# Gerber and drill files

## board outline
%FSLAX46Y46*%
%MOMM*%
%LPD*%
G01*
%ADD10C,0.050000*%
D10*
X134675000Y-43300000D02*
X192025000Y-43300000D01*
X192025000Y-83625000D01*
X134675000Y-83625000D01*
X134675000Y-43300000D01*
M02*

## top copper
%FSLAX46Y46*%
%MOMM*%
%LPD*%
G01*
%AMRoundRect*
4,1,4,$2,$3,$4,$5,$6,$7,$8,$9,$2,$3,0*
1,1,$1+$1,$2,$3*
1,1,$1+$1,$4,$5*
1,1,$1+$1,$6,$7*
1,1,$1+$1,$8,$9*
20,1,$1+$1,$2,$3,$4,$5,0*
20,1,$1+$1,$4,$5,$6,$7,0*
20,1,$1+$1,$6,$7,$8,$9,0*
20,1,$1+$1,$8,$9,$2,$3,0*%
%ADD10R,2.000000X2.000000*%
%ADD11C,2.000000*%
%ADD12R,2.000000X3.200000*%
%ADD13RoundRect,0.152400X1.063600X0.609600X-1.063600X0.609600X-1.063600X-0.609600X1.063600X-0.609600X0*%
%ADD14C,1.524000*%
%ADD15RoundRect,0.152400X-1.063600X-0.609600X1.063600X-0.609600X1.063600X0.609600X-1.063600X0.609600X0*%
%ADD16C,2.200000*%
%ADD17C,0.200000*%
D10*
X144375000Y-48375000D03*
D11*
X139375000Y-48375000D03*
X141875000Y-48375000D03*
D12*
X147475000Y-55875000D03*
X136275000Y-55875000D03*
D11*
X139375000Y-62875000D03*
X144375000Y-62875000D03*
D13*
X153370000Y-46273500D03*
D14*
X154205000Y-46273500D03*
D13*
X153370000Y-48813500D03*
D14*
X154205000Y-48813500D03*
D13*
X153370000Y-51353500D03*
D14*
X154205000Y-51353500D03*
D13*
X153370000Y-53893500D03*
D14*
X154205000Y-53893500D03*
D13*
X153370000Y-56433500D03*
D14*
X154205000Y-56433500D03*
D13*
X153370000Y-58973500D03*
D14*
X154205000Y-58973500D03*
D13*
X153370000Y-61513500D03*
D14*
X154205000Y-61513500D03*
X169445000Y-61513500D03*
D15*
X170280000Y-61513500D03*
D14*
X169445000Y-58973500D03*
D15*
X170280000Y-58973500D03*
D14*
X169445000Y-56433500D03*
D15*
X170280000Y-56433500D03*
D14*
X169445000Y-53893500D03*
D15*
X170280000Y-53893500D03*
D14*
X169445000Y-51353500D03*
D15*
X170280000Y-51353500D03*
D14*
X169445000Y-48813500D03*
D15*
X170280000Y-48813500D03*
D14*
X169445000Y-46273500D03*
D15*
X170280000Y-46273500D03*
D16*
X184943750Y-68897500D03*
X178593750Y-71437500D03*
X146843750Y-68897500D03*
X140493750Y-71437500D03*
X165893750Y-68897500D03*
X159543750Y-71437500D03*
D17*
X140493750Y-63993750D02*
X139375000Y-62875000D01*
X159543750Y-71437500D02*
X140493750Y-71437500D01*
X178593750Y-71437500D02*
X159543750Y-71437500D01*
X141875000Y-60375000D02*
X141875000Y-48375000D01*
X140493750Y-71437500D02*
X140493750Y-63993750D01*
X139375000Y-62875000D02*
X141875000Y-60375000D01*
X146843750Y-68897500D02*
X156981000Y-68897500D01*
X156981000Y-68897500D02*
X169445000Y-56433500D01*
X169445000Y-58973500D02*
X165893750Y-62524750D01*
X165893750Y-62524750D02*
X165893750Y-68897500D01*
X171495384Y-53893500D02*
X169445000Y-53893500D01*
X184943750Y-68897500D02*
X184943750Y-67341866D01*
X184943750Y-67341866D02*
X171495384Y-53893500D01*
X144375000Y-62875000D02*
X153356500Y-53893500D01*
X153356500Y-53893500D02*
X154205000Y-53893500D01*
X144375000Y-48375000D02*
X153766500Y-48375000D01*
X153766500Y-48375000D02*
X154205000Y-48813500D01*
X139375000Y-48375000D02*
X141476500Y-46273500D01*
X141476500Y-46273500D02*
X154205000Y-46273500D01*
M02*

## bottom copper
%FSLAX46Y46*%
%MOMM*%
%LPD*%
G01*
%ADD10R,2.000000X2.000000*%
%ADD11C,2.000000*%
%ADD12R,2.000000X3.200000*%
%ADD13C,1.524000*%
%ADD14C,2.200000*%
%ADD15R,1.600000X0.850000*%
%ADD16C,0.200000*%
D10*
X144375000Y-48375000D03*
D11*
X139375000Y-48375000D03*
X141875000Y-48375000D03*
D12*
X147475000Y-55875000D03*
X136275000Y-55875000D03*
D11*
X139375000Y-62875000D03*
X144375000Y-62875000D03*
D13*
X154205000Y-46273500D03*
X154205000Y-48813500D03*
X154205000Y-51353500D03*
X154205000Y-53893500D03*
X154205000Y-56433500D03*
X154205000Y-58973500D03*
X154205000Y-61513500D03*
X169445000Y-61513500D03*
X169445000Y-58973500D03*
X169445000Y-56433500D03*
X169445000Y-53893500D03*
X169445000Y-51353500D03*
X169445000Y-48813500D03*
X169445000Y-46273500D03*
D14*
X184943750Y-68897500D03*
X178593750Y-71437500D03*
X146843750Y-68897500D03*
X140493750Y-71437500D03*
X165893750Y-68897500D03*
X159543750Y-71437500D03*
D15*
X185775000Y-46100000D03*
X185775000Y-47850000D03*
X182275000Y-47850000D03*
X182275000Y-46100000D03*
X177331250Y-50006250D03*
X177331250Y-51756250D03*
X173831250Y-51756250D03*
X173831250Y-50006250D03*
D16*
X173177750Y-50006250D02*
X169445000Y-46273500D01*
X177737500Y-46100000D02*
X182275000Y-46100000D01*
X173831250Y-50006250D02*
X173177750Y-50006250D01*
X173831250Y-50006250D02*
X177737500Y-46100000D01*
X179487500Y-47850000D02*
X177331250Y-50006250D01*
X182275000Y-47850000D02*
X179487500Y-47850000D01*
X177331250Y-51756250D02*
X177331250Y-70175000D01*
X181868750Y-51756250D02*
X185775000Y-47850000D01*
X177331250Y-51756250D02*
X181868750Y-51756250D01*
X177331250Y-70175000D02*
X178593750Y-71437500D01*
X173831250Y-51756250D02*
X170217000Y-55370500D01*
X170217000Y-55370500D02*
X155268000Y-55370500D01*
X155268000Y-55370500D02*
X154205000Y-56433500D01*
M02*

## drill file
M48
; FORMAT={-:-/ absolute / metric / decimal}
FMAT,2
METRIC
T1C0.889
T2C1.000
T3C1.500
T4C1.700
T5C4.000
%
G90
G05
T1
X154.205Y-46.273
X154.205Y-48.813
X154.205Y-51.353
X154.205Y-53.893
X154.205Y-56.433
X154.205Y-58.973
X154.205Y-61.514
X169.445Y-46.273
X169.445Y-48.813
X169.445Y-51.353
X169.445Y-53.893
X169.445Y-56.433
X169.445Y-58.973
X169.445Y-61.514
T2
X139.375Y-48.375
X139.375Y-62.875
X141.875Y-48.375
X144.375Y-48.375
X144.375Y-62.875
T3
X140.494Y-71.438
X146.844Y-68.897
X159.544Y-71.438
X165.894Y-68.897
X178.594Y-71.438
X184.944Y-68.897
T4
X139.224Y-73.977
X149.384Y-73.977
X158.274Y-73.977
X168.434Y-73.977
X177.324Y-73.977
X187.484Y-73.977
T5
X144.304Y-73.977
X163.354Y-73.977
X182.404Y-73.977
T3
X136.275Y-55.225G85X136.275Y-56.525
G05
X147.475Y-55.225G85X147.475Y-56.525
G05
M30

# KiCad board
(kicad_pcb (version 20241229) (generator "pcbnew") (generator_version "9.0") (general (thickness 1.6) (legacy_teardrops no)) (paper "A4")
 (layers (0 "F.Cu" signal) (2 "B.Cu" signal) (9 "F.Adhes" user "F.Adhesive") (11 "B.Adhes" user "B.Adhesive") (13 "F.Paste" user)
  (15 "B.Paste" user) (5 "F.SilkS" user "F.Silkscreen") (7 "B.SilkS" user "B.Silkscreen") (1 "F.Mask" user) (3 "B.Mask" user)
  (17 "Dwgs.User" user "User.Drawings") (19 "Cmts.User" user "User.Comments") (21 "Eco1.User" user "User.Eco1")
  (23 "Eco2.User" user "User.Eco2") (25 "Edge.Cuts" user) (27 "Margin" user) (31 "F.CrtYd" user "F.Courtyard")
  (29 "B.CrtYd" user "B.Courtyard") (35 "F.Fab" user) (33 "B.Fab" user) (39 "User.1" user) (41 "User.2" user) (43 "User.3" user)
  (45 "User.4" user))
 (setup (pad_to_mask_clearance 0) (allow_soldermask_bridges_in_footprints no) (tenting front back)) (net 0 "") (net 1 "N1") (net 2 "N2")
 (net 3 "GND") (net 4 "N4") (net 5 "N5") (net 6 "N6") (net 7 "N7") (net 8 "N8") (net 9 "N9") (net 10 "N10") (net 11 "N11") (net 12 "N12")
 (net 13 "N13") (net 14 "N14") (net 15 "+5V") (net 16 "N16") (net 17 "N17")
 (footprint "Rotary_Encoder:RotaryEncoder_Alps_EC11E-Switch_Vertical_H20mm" (layer "F.Cu") (at 144.375 48.375 -90)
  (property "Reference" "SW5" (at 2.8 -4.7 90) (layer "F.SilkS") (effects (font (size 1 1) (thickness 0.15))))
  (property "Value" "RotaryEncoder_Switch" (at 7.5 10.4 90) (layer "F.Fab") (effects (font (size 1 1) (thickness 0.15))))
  (pad "A" thru_hole rect (at 0 0 270) (size 2 2) (drill 1) (layers "*.Cu" "*.Mask") (remove_unused_layers no) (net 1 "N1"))
  (pad "B" thru_hole circle (at 0 5 270) (size 2 2) (drill 1) (layers "*.Cu" "*.Mask") (remove_unused_layers no) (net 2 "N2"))
  (pad "C" thru_hole circle (at 0 2.5 270) (size 2 2) (drill 1) (layers "*.Cu" "*.Mask") (remove_unused_layers no) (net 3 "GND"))
  (pad "MP" thru_hole rect (at 7.5 -3.1 270) (size 3.2 2) (drill oval 2.8 1.5) (layers "*.Cu" "*.Mask") (remove_unused_layers no))
  (pad "MP" thru_hole rect (at 7.5 8.1 270) (size 3.2 2) (drill oval 2.8 1.5) (layers "*.Cu" "*.Mask") (remove_unused_layers no))
  (pad "S1" thru_hole circle (at 14.5 5 270) (size 2 2) (drill 1) (layers "*.Cu" "*.Mask") (remove_unused_layers no) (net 3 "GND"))
  (pad "S2" thru_hole circle (at 14.5 0 270) (size 2 2) (drill 1) (layers "*.Cu" "*.Mask") (remove_unused_layers no) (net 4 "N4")))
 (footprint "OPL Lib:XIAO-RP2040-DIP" (layer "F.Cu") (at 161.825 53.8935)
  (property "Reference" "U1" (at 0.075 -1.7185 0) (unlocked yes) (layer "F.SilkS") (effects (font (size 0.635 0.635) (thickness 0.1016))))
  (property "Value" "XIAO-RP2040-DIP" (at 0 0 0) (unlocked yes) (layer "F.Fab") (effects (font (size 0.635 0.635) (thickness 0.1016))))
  (pad "1" smd roundrect (at -8.455 -7.62 180) (size 2.432 1.524) (layers "F.Cu" "F.Mask") (roundrect_rratio 0.1) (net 2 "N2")
   (thermal_bridge_angle 45))
  (pad "1" thru_hole circle (at -7.62 -7.62 180) (size 1.524 1.524) (drill 0.889) (layers "*.Cu" "*.Mask") (remove_unused_layers no)
   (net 2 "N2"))
  (pad "2" smd roundrect (at -8.455 -5.08 180) (size 2.432 1.524) (layers "F.Cu" "F.Mask") (roundrect_rratio 0.1) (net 1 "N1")
   (thermal_bridge_angle 45))
  (pad "2" thru_hole circle (at -7.62 -5.08 180) (size 1.524 1.524) (drill 0.889) (layers "*.Cu" "*.Mask") (remove_unused_layers no)
   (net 1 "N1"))
  (pad "3" smd roundrect (at -8.455 -2.54 180) (size 2.432 1.524) (layers "F.Cu" "F.Mask") (roundrect_rratio 0.1) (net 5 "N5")
   (thermal_bridge_angle 45))
  (pad "3" thru_hole circle (at -7.62 -2.54 180) (size 1.524 1.524) (drill 0.889) (layers "*.Cu" "*.Mask") (remove_unused_layers no)
   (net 5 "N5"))
  (pad "4" smd roundrect (at -8.455 0 180) (size 2.432 1.524) (layers "F.Cu" "F.Mask") (roundrect_rratio 0.1) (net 4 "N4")
   (thermal_bridge_angle 45))
  (pad "4" thru_hole circle (at -7.62 0 180) (size 1.524 1.524) (drill 0.889) (layers "*.Cu" "*.Mask") (remove_unused_layers no)
   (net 4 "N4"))
  (pad "5" smd roundrect (at -8.455 2.54 180) (size 2.432 1.524) (layers "F.Cu" "F.Mask") (roundrect_rratio 0.1) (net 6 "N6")
   (thermal_bridge_angle 45))
  (pad "5" thru_hole circle (at -7.62 2.54 180) (size 1.524 1.524) (drill 0.889) (layers "*.Cu" "*.Mask") (remove_unused_layers no)
   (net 6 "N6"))
  (pad "6" smd roundrect (at -8.455 5.08 180) (size 2.432 1.524) (layers "F.Cu" "F.Mask") (roundrect_rratio 0.1) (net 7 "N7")
   (thermal_bridge_angle 45))
  (pad "6" thru_hole circle (at -7.62 5.08 180) (size 1.524 1.524) (drill 0.889) (layers "*.Cu" "*.Mask") (remove_unused_layers no)
   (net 7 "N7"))
  (pad "7" smd roundrect (at -8.455 7.62 180) (size 2.432 1.524) (layers "F.Cu" "F.Mask") (roundrect_rratio 0.1) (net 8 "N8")
   (thermal_bridge_angle 45))
  (pad "7" thru_hole circle (at -7.62 7.62 180) (size 1.524 1.524) (drill 0.889) (layers "*.Cu" "*.Mask") (remove_unused_layers no)
   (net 8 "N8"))
  (pad "8" thru_hole circle (at 7.62 7.62) (size 1.524 1.524) (drill 0.889) (layers "*.Cu" "*.Mask") (remove_unused_layers no) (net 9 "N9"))
  (pad "8" smd roundrect (at 8.455 7.62) (size 2.432 1.524) (layers "F.Cu" "F.Mask") (roundrect_rratio 0.1) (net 9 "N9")
   (thermal_bridge_angle 45))
  (pad "9" thru_hole circle (at 7.62 5.08) (size 1.524 1.524) (drill 0.889) (layers "*.Cu" "*.Mask") (remove_unused_layers no)
   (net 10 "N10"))
  (pad "9" smd roundrect (at 8.455 5.08) (size 2.432 1.524) (layers "F.Cu" "F.Mask") (roundrect_rratio 0.1) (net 10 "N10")
   (thermal_bridge_angle 45))
  (pad "10" thru_hole circle (at 7.62 2.54) (size 1.524 1.524) (drill 0.889) (layers "*.Cu" "*.Mask") (remove_unused_layers no)
   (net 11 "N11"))
  (pad "10" smd roundrect (at 8.455 2.54) (size 2.432 1.524) (layers "F.Cu" "F.Mask") (roundrect_rratio 0.1) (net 11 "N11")
   (thermal_bridge_angle 45))
  (pad "11" thru_hole circle (at 7.62 0) (size 1.524 1.524) (drill 0.889) (layers "*.Cu" "*.Mask") (remove_unused_layers no) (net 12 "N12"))
  (pad "11" smd roundrect (at 8.455 0) (size 2.432 1.524) (layers "F.Cu" "F.Mask") (roundrect_rratio 0.1) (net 12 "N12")
   (thermal_bridge_angle 45))
  (pad "12" thru_hole circle (at 7.62 -2.54) (size 1.524 1.524) (drill 0.889) (layers "*.Cu" "*.Mask") (remove_unused_layers no)
   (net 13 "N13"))
  (pad "12" smd roundrect (at 8.455 -2.54) (size 2.432 1.524) (layers "F.Cu" "F.Mask") (roundrect_rratio 0.1) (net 13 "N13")
   (thermal_bridge_angle 45))
  (pad "13" thru_hole circle (at 7.62 -5.08) (size 1.524 1.524) (drill 0.889) (layers "*.Cu" "*.Mask") (remove_unused_layers no)
   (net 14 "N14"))
  (pad "13" smd roundrect (at 8.455 -5.08) (size 2.432 1.524) (layers "F.Cu" "F.Mask") (roundrect_rratio 0.1) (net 14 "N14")
   (thermal_bridge_angle 45))
  (pad "14" thru_hole circle (at 7.62 -7.62) (size 1.524 1.524) (drill 0.889) (layers "*.Cu" "*.Mask") (remove_unused_layers no)
   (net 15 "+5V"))
  (pad "14" smd roundrect (at 8.455 -7.62) (size 2.432 1.524) (layers "F.Cu" "F.Mask") (roundrect_rratio 0.1) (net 15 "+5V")
   (thermal_bridge_angle 45)))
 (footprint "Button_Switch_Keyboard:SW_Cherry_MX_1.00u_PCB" (layer "F.Cu") (at 184.94375 68.8975)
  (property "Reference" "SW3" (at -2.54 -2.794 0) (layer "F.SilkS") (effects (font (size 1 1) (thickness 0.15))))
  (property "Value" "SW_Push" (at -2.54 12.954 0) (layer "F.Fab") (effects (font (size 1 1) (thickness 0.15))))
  (pad "" np_thru_hole circle (at -7.62 5.08) (size 1.7 1.7) (drill 1.7) (layers "*.Cu" "*.Mask"))
  (pad "" np_thru_hole circle (at -2.54 5.08) (size 4 4) (drill 4) (layers "*.Cu" "*.Mask"))
  (pad "" np_thru_hole circle (at 2.54 5.08) (size 1.7 1.7) (drill 1.7) (layers "*.Cu" "*.Mask"))
  (pad "1" thru_hole circle (at 0 0) (size 2.2 2.2) (drill 1.5) (layers "*.Cu" "*.Mask") (remove_unused_layers no) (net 12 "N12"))
  (pad "2" thru_hole circle (at -6.35 2.54) (size 2.2 2.2) (drill 1.5) (layers "*.Cu" "*.Mask") (remove_unused_layers no) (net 3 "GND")))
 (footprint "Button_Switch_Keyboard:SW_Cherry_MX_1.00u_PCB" (layer "F.Cu") (at 146.84375 68.8975)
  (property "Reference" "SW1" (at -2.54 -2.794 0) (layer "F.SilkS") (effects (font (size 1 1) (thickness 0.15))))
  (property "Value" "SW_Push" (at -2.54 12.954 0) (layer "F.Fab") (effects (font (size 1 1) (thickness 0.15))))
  (pad "" np_thru_hole circle (at -7.62 5.08) (size 1.7 1.7) (drill 1.7) (layers "*.Cu" "*.Mask"))
  (pad "" np_thru_hole circle (at -2.54 5.08) (size 4 4) (drill 4) (layers "*.Cu" "*.Mask"))
  (pad "" np_thru_hole circle (at 2.54 5.08) (size 1.7 1.7) (drill 1.7) (layers "*.Cu" "*.Mask"))
  (pad "1" thru_hole circle (at 0 0) (size 2.2 2.2) (drill 1.5) (layers "*.Cu" "*.Mask") (remove_unused_layers no) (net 11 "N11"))
  (pad "2" thru_hole circle (at -6.35 2.54) (size 2.2 2.2) (drill 1.5) (layers "*.Cu" "*.Mask") (remove_unused_layers no) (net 3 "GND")))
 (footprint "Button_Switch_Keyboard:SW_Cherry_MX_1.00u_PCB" (layer "F.Cu") (at 165.89375 68.8975)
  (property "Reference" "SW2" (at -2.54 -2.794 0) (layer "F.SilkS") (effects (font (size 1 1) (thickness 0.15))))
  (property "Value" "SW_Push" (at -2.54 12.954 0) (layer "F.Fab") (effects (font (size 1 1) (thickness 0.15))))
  (pad "" np_thru_hole circle (at -7.62 5.08) (size 1.7 1.7) (drill 1.7) (layers "*.Cu" "*.Mask"))
  (pad "" np_thru_hole circle (at -2.54 5.08) (size 4 4) (drill 4) (layers "*.Cu" "*.Mask"))
  (pad "" np_thru_hole circle (at 2.54 5.08) (size 1.7 1.7) (drill 1.7) (layers "*.Cu" "*.Mask"))
  (pad "1" thru_hole circle (at 0 0) (size 2.2 2.2) (drill 1.5) (layers "*.Cu" "*.Mask") (remove_unused_layers no) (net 10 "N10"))
  (pad "2" thru_hole circle (at -6.35 2.54) (size 2.2 2.2) (drill 1.5) (layers "*.Cu" "*.Mask") (remove_unused_layers no) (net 3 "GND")))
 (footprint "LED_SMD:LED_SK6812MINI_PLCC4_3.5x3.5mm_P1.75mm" (layer "B.Cu") (at 184.025 46.975 180)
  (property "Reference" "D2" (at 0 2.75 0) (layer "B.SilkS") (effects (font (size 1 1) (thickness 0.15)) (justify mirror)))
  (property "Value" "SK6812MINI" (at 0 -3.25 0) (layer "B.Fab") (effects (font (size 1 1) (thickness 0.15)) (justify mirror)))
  (pad "1" smd rect (at -1.75 0.875 180) (size 1.6 0.85) (layers "B.Cu" "B.Mask" "B.Paste") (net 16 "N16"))
  (pad "2" smd rect (at -1.75 -0.875 180) (size 1.6 0.85) (layers "B.Cu" "B.Mask" "B.Paste") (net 3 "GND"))
  (pad "3" smd rect (at 1.75 -0.875 180) (size 1.6 0.85) (layers "B.Cu" "B.Mask" "B.Paste") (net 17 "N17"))
  (pad "4" smd rect (at 1.75 0.875 180) (size 1.6 0.85) (layers "B.Cu" "B.Mask" "B.Paste") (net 15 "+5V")))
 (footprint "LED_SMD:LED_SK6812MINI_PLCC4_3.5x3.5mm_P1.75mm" (layer "B.Cu") (at 175.58125 50.88125 180)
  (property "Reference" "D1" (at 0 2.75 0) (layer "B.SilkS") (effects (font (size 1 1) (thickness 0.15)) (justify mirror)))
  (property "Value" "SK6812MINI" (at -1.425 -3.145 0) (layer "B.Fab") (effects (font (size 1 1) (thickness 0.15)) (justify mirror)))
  (pad "1" smd rect (at -1.75 0.875 180) (size 1.6 0.85) (layers "B.Cu" "B.Mask" "B.Paste") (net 17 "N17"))
  (pad "2" smd rect (at -1.75 -0.875 180) (size 1.6 0.85) (layers "B.Cu" "B.Mask" "B.Paste") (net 3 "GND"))
  (pad "3" smd rect (at 1.75 -0.875 180) (size 1.6 0.85) (layers "B.Cu" "B.Mask" "B.Paste") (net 6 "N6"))
  (pad "4" smd rect (at 1.75 0.875 180) (size 1.6 0.85) (layers "B.Cu" "B.Mask" "B.Paste") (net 15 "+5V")))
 (gr_rect (start 134.675 43.3) (end 192.025 83.625) (stroke (width 0.05) (type default)) (fill no) (layer "Edge.Cuts"))
 (segment (start 173.17775 50.00625) (end 169.445 46.2735) (width 0.2) (layer "B.Cu") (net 15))
 (segment (start 177.7375 46.1) (end 182.275 46.1) (width 0.2) (layer "B.Cu") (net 15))
 (segment (start 173.83125 50.00625) (end 173.17775 50.00625) (width 0.2) (layer "B.Cu") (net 15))
 (segment (start 173.83125 50.00625) (end 177.7375 46.1) (width 0.2) (layer "B.Cu") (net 15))
 (segment (start 179.4875 47.85) (end 177.33125 50.00625) (width 0.2) (layer "B.Cu") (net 17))
 (segment (start 182.275 47.85) (end 179.4875 47.85) (width 0.2) (layer "B.Cu") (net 17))
 (segment (start 140.49375 63.99375) (end 139.375 62.875) (width 0.2) (layer "F.Cu") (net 3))
 (segment (start 159.54375 71.4375) (end 140.49375 71.4375) (width 0.2) (layer "F.Cu") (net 3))
 (segment (start 178.59375 71.4375) (end 159.54375 71.4375) (width 0.2) (layer "F.Cu") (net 3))
 (segment (start 141.875 60.375) (end 141.875 48.375) (width 0.2) (layer "F.Cu") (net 3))
 (segment (start 140.49375 71.4375) (end 140.49375 63.99375) (width 0.2) (layer "F.Cu") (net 3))
 (segment (start 139.375 62.875) (end 141.875 60.375) (width 0.2) (layer "F.Cu") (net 3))
 (segment (start 177.33125 51.75625) (end 177.33125 70.175) (width 0.2) (layer "B.Cu") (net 3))
 (segment (start 181.86875 51.75625) (end 185.775 47.85) (width 0.2) (layer "B.Cu") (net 3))
 (segment (start 177.33125 51.75625) (end 181.86875 51.75625) (width 0.2) (layer "B.Cu") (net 3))
 (segment (start 177.33125 70.175) (end 178.59375 71.4375) (width 0.2) (layer "B.Cu") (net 3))
 (segment (start 173.83125 51.75625) (end 170.217 55.3705) (width 0.2) (layer "B.Cu") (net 6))
 (segment (start 170.217 55.3705) (end 155.268 55.3705) (width 0.2) (layer "B.Cu") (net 6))
 (segment (start 155.268 55.3705) (end 154.205 56.4335) (width 0.2) (layer "B.Cu") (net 6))
 (segment (start 146.84375 68.8975) (end 156.981 68.8975) (width 0.2) (layer "F.Cu") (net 11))
 (segment (start 156.981 68.8975) (end 169.445 56.4335) (width 0.2) (layer "F.Cu") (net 11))
 (segment (start 169.445 58.9735) (end 165.89375 62.52475) (width 0.2) (layer "F.Cu") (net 10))
 (segment (start 165.89375 62.52475) (end 165.89375 68.8975) (width 0.2) (layer "F.Cu") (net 10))
 (segment (start 171.495384 53.8935) (end 169.445 53.8935) (width 0.2) (layer "F.Cu") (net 12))
 (segment (start 184.94375 68.8975) (end 184.94375 67.341866) (width 0.2) (layer "F.Cu") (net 12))
 (segment (start 184.94375 67.341866) (end 171.495384 53.8935) (width 0.2) (layer "F.Cu") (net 12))
 (segment (start 144.375 62.875) (end 153.3565 53.8935) (width 0.2) (layer "F.Cu") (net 4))
 (segment (start 153.3565 53.8935) (end 154.205 53.8935) (width 0.2) (layer "F.Cu") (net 4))
 (segment (start 144.375 48.375) (end 153.7665 48.375) (width 0.2) (layer "F.Cu") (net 1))
 (segment (start 153.7665 48.375) (end 154.205 48.8135) (width 0.2) (layer "F.Cu") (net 1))
 (segment (start 139.375 48.375) (end 141.4765 46.2735) (width 0.2) (layer "F.Cu") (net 2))
 (segment (start 141.4765 46.2735) (end 154.205 46.2735) (width 0.2) (layer "F.Cu") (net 2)))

